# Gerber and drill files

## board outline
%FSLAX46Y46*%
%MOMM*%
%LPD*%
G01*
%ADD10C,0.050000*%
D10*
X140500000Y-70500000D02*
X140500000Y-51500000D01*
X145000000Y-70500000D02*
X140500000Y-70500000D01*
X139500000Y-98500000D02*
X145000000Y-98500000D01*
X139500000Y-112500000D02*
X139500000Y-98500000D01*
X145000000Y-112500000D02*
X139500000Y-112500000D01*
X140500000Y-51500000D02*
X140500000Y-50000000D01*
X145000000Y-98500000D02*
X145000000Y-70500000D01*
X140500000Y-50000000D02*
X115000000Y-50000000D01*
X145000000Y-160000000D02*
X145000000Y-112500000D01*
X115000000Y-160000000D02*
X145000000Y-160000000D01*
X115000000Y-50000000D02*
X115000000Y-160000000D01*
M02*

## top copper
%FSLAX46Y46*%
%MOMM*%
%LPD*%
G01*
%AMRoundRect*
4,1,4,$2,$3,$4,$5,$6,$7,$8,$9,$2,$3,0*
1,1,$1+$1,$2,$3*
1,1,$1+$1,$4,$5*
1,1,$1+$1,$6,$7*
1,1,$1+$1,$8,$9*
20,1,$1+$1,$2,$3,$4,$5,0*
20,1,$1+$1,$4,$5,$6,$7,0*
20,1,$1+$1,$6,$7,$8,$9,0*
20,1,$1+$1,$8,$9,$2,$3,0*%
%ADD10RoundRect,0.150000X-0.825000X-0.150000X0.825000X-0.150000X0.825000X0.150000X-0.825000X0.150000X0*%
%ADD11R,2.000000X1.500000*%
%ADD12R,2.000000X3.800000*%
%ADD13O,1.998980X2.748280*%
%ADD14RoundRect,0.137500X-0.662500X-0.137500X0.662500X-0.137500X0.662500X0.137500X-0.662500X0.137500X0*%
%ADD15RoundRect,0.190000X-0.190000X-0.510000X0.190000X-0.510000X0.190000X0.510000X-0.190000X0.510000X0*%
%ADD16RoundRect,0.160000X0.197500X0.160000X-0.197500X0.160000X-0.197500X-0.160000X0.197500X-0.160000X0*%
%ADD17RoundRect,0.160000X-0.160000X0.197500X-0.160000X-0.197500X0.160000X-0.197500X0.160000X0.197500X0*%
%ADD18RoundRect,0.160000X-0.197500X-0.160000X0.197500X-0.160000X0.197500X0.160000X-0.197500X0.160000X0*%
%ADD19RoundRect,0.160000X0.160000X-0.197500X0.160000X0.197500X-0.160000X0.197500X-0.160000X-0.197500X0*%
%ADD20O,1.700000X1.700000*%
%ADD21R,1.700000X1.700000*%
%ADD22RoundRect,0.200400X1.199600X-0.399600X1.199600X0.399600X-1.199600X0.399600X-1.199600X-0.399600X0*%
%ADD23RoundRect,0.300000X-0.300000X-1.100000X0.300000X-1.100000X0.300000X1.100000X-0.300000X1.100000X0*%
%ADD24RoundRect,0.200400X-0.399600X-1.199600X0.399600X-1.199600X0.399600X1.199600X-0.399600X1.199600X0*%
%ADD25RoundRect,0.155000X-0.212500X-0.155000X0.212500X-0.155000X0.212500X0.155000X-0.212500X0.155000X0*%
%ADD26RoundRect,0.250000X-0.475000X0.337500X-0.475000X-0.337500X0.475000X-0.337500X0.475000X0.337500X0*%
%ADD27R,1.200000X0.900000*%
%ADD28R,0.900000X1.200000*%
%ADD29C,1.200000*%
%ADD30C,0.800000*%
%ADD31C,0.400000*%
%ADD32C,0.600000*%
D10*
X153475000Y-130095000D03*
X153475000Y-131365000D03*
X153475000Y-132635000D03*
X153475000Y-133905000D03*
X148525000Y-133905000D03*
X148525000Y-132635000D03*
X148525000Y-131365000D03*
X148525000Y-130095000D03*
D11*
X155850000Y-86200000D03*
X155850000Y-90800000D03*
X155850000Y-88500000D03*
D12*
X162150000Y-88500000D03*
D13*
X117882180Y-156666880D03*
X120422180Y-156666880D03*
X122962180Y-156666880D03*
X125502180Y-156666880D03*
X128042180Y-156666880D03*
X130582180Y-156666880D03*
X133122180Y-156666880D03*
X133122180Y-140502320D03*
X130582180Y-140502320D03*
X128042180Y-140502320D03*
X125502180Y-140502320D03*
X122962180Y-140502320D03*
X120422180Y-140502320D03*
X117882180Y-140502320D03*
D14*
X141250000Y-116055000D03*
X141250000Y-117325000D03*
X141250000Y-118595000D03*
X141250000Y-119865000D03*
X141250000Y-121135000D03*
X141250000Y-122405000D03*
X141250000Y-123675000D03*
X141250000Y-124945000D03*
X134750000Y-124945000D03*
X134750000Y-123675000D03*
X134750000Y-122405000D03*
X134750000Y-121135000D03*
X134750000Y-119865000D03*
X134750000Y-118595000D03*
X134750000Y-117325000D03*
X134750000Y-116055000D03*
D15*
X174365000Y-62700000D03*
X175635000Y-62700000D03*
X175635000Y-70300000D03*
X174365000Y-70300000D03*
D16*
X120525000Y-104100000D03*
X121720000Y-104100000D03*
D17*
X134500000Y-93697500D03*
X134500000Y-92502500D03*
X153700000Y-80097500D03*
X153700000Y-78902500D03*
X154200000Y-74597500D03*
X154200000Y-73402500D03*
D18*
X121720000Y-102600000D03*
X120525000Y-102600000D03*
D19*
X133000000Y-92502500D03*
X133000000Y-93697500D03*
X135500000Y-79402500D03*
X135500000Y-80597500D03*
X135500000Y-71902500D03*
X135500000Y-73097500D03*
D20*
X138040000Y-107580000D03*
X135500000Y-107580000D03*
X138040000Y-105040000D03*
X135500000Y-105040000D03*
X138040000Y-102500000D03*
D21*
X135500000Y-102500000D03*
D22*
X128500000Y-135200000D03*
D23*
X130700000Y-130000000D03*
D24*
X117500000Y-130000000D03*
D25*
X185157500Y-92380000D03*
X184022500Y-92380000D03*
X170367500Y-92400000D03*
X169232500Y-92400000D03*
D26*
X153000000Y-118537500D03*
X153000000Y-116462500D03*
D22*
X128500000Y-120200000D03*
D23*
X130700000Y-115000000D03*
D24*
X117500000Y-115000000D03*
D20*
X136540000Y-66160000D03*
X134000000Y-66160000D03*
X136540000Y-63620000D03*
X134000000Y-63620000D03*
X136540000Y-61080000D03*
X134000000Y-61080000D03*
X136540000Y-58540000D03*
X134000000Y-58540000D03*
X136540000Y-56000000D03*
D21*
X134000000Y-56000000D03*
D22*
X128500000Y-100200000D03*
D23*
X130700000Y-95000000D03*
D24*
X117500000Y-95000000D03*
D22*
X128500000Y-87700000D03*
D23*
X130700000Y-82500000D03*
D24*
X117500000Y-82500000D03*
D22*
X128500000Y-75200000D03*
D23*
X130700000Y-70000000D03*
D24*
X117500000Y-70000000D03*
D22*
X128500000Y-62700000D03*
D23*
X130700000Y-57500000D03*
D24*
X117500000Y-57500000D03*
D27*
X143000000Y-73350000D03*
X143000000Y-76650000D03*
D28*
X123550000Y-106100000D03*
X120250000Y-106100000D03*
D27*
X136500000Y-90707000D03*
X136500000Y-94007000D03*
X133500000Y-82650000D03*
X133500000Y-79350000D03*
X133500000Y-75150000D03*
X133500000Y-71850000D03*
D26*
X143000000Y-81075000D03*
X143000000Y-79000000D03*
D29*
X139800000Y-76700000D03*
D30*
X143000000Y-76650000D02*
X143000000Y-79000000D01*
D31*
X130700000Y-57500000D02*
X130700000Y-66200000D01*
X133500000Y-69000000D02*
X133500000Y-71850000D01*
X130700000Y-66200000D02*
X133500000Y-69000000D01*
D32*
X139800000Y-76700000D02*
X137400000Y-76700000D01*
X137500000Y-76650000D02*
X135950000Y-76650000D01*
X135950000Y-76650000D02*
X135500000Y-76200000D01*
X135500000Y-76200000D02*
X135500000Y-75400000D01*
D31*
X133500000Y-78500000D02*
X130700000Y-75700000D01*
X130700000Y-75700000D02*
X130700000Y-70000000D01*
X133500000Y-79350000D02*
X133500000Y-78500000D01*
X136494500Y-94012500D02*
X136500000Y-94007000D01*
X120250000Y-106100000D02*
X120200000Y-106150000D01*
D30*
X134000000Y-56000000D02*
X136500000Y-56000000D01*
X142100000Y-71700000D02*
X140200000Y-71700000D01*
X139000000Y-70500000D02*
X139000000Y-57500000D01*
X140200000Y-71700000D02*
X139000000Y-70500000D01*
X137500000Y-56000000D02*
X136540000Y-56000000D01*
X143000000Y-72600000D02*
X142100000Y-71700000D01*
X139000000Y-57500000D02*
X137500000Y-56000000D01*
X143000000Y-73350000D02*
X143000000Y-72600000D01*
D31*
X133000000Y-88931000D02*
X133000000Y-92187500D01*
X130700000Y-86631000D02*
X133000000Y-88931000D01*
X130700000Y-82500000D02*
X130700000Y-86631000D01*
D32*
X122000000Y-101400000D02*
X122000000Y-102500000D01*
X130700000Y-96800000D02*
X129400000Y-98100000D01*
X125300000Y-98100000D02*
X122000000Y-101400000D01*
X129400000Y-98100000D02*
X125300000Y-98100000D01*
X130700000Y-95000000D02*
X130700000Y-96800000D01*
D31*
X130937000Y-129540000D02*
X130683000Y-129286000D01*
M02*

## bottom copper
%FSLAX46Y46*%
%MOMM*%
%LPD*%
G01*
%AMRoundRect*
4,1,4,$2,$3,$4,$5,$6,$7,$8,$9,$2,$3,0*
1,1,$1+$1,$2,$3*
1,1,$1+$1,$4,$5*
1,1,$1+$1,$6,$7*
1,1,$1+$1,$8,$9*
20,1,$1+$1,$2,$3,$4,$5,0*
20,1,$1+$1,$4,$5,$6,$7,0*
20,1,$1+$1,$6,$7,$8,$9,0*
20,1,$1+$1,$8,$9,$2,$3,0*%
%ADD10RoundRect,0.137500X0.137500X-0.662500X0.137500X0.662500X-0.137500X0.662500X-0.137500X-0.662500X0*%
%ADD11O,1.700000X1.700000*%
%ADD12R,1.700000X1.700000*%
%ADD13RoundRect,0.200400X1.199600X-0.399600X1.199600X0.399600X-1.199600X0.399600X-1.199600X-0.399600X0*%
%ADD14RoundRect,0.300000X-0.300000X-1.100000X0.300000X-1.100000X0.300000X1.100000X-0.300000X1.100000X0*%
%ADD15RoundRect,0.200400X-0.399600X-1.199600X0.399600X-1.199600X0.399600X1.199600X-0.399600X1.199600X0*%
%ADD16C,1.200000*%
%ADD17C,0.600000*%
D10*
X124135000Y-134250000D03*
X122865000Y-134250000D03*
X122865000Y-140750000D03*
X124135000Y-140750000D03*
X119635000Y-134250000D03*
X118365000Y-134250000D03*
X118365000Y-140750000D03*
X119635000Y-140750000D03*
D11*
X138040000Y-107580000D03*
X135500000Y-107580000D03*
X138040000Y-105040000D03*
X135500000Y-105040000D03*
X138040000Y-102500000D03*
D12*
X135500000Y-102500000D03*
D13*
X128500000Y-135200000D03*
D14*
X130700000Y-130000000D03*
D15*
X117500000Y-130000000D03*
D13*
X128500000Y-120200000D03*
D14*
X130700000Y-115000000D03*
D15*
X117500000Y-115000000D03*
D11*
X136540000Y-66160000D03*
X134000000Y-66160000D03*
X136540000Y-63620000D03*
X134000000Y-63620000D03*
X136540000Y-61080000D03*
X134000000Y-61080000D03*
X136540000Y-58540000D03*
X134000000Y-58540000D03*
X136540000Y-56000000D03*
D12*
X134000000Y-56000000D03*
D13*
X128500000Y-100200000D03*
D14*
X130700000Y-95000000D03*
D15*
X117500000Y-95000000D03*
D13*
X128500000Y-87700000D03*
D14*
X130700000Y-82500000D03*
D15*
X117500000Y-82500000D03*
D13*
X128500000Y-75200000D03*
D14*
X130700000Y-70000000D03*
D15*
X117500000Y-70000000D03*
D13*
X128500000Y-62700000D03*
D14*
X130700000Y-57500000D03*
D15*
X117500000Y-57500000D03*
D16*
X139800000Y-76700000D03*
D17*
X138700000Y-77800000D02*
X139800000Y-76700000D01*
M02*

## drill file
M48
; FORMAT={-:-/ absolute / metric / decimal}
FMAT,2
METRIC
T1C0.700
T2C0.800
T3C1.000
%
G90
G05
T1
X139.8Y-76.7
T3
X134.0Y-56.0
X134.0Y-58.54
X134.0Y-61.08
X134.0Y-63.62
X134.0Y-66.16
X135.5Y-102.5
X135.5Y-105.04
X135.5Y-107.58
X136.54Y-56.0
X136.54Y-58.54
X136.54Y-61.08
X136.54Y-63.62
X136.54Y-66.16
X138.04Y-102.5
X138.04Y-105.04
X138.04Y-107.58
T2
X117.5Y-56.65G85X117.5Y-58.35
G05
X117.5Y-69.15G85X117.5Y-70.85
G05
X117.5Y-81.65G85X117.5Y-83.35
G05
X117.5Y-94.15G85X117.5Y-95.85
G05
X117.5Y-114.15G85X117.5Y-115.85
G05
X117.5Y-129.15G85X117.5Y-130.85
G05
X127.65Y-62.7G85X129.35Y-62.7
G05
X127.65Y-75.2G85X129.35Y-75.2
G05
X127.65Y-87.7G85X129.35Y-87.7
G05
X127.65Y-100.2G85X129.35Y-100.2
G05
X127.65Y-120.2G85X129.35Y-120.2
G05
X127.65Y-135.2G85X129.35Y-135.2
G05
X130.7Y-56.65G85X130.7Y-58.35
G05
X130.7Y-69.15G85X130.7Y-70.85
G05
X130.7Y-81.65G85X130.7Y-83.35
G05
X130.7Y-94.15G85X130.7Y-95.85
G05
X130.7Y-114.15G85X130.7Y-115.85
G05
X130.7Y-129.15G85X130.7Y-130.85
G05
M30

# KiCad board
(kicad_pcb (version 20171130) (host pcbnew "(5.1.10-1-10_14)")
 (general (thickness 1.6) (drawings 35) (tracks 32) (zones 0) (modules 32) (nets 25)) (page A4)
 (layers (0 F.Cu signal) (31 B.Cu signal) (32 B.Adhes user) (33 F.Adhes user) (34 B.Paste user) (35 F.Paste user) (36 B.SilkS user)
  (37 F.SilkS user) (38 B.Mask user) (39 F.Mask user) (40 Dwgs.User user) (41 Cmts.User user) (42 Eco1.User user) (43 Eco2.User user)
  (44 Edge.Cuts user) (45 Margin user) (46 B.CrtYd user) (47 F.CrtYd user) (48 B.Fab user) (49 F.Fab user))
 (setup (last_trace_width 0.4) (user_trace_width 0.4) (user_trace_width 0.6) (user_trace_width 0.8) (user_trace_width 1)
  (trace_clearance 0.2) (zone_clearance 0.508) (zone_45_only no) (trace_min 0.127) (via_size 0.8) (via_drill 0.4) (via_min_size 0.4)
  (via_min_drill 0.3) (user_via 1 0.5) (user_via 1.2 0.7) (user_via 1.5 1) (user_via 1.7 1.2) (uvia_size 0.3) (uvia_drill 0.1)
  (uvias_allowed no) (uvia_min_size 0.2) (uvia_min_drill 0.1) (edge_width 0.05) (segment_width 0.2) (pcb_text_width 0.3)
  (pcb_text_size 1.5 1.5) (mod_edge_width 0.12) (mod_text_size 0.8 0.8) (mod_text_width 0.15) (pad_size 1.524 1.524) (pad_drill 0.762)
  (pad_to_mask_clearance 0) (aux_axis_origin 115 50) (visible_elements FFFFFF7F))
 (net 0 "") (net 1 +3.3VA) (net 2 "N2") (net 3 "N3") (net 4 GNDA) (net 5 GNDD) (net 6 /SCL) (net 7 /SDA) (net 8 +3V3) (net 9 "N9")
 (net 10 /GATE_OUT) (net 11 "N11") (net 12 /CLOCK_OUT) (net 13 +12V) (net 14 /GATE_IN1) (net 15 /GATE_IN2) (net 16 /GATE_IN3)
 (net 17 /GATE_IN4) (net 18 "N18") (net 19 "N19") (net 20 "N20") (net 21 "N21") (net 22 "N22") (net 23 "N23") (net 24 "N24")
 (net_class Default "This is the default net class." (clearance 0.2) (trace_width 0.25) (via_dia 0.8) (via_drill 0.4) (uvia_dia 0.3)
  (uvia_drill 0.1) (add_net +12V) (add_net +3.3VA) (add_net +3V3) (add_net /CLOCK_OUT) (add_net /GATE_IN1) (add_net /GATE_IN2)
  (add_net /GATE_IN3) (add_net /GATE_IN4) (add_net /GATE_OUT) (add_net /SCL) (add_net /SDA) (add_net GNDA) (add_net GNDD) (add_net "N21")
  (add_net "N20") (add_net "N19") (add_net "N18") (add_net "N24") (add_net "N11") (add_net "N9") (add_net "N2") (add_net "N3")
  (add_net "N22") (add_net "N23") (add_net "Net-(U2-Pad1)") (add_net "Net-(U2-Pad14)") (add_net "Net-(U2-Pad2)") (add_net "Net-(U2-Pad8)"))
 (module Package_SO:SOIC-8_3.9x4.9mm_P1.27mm (layer F.Cu) (at 151 132)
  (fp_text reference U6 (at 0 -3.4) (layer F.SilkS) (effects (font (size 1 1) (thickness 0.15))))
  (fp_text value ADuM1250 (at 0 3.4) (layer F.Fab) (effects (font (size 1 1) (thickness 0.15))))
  (pad 8 smd roundrect (at 2.475 -1.905) (size 1.95 0.6) (layers F.Cu F.Paste F.Mask) (roundrect_rratio 0.25) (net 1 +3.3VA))
  (pad 7 smd roundrect (at 2.475 -0.635) (size 1.95 0.6) (layers F.Cu F.Paste F.Mask) (roundrect_rratio 0.25) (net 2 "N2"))
  (pad 6 smd roundrect (at 2.475 0.635) (size 1.95 0.6) (layers F.Cu F.Paste F.Mask) (roundrect_rratio 0.25) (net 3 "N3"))
  (pad 5 smd roundrect (at 2.475 1.905) (size 1.95 0.6) (layers F.Cu F.Paste F.Mask) (roundrect_rratio 0.25) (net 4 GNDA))
  (pad 4 smd roundrect (at -2.475 1.905) (size 1.95 0.6) (layers F.Cu F.Paste F.Mask) (roundrect_rratio 0.25) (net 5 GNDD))
  (pad 3 smd roundrect (at -2.475 0.635) (size 1.95 0.6) (layers F.Cu F.Paste F.Mask) (roundrect_rratio 0.25) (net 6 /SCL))
  (pad 2 smd roundrect (at -2.475 -0.635) (size 1.95 0.6) (layers F.Cu F.Paste F.Mask) (roundrect_rratio 0.25) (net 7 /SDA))
  (pad 1 smd roundrect (at -2.475 -1.905) (size 1.95 0.6) (layers F.Cu F.Paste F.Mask) (roundrect_rratio 0.25) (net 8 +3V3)))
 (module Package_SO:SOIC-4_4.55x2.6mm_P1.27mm (layer B.Cu) (at 123.5 137.5 90)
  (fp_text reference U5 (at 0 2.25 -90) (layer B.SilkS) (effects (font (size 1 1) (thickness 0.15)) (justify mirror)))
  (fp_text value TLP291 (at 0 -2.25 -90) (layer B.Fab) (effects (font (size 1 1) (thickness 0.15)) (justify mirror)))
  (pad 4 smd roundrect (at 3.25 0.635 90) (size 1.6 0.55) (layers B.Cu B.Paste B.Mask) (roundrect_rratio 0.25) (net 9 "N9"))
  (pad 3 smd roundrect (at 3.25 -0.635 90) (size 1.6 0.55) (layers B.Cu B.Paste B.Mask) (roundrect_rratio 0.25) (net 4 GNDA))
  (pad 2 smd roundrect (at -3.25 -0.635 90) (size 1.6 0.55) (layers B.Cu B.Paste B.Mask) (roundrect_rratio 0.25) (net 5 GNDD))
  (pad 1 smd roundrect (at -3.25 0.635 90) (size 1.6 0.55) (layers B.Cu B.Paste B.Mask) (roundrect_rratio 0.25) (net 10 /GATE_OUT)))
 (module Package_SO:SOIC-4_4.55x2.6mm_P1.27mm (layer B.Cu) (at 119 137.5 90)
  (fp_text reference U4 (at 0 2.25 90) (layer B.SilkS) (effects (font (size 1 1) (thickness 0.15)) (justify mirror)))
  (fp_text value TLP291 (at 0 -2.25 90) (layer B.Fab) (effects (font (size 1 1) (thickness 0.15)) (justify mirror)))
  (pad 4 smd roundrect (at 3.25 0.635 90) (size 1.6 0.55) (layers B.Cu B.Paste B.Mask) (roundrect_rratio 0.25) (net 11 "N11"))
  (pad 3 smd roundrect (at 3.25 -0.635 90) (size 1.6 0.55) (layers B.Cu B.Paste B.Mask) (roundrect_rratio 0.25) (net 4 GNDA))
  (pad 2 smd roundrect (at -3.25 -0.635 90) (size 1.6 0.55) (layers B.Cu B.Paste B.Mask) (roundrect_rratio 0.25) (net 5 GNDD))
  (pad 1 smd roundrect (at -3.25 0.635 90) (size 1.6 0.55) (layers B.Cu B.Paste B.Mask) (roundrect_rratio 0.25) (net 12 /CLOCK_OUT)))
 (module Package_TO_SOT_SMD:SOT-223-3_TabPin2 (layer F.Cu) (at 159 88.5)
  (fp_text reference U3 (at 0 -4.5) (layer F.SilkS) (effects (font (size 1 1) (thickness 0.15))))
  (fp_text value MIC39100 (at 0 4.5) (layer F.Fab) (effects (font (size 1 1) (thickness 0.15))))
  (pad 1 smd rect (at -3.15 -2.3) (size 2 1.5) (layers F.Cu F.Paste F.Mask) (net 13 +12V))
  (pad 3 smd rect (at -3.15 2.3) (size 2 1.5) (layers F.Cu F.Paste F.Mask) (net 1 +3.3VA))
  (pad 2 smd rect (at -3.15 0) (size 2 1.5) (layers F.Cu F.Paste F.Mask) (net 4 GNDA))
  (pad 2 smd rect (at 3.15 0) (size 2 3.8) (layers F.Cu F.Paste F.Mask) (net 4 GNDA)))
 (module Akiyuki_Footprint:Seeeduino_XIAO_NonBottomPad (layer F.Cu) (at 136 157.5 90)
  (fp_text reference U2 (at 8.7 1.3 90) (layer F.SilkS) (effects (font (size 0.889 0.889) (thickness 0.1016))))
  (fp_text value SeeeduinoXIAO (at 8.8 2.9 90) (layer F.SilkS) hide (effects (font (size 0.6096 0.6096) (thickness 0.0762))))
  (pad "" smd circle (at 10.238803 -16.264187 180) (size 1.143 1.143) (layers Dwgs.User))
  (pad "" smd circle (at 7.698803 -16.264187 180) (size 1.143 1.143) (layers Dwgs.User))
  (pad "" smd circle (at 10.238803 -18.804187 180) (size 1.143 1.143) (layers Dwgs.User))
  (pad "" smd circle (at 7.698803 -18.804187 180) (size 1.143 1.143) (layers Dwgs.User))
  (pad "" smd oval (at 10.25 -1.8 180) (size 2.032 1.016) (layers Dwgs.User))
  (pad "" smd oval (at 7.7 -1.8 180) (size 2.032 1.016) (layers Dwgs.User))
  (pad 1 smd oval (at 0.83312 -18.11782 90) (size 2.74828 1.99898) (layers F.Cu F.Paste F.Mask))
  (pad 2 smd oval (at 0.83312 -15.57782 90) (size 2.74828 1.99898) (layers F.Cu F.Paste F.Mask))
  (pad 3 smd oval (at 0.83312 -13.03782 90) (size 2.74828 1.99898) (layers F.Cu F.Paste F.Mask) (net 12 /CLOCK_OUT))
  (pad 4 smd oval (at 0.83312 -10.49782 90) (size 2.74828 1.99898) (layers F.Cu F.Paste F.Mask) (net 10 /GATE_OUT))
  (pad 5 smd oval (at 0.83312 -7.95782 90) (size 2.74828 1.99898) (layers F.Cu F.Paste F.Mask) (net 7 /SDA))
  (pad 6 smd oval (at 0.83312 -5.41782 90) (size 2.74828 1.99898) (layers F.Cu F.Paste F.Mask) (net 6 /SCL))
  (pad 7 smd oval (at 0.83312 -2.87782 90) (size 2.74828 1.99898) (layers F.Cu F.Paste F.Mask) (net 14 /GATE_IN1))
  (pad 8 smd oval (at 16.99768 -2.87782 90) (size 2.74828 1.99898) (layers F.Cu F.Paste F.Mask))
  (pad 9 smd oval (at 16.99768 -5.41782 90) (size 2.74828 1.99898) (layers F.Cu F.Paste F.Mask) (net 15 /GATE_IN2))
  (pad 10 smd oval (at 16.99768 -7.95782 90) (size 2.74828 1.99898) (layers F.Cu F.Paste F.Mask) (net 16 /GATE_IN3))
  (pad 11 smd oval (at 16.99768 -10.49782 90) (size 2.74828 1.99898) (layers F.Cu F.Paste F.Mask) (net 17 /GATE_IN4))
  (pad 12 smd oval (at 16.99768 -13.03782 90) (size 2.74828 1.99898) (layers F.Cu F.Paste F.Mask) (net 8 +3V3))
  (pad 13 smd oval (at 16.99768 -15.57782 90) (size 2.74828 1.99898) (layers F.Cu F.Paste F.Mask) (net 5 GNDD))
  (pad 14 smd oval (at 16.99768 -18.11782 90) (size 2.74828 1.99898) (layers F.Cu F.Paste F.Mask)))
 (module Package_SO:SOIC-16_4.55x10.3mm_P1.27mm (layer F.Cu) (at 138 120.5)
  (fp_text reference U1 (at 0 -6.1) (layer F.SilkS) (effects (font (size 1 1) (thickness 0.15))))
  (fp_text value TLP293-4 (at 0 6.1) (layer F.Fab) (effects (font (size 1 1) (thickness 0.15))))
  (pad 16 smd roundrect (at 3.25 -4.445) (size 1.6 0.55) (layers F.Cu F.Paste F.Mask) (roundrect_rratio 0.25) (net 14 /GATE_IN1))
  (pad 15 smd roundrect (at 3.25 -3.175) (size 1.6 0.55) (layers F.Cu F.Paste F.Mask) (roundrect_rratio 0.25) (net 5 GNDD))
  (pad 14 smd roundrect (at 3.25 -1.905) (size 1.6 0.55) (layers F.Cu F.Paste F.Mask) (roundrect_rratio 0.25) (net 15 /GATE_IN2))
  (pad 13 smd roundrect (at 3.25 -0.635) (size 1.6 0.55) (layers F.Cu F.Paste F.Mask) (roundrect_rratio 0.25) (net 5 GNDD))
  (pad 12 smd roundrect (at 3.25 0.635) (size 1.6 0.55) (layers F.Cu F.Paste F.Mask) (roundrect_rratio 0.25) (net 16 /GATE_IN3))
  (pad 11 smd roundrect (at 3.25 1.905) (size 1.6 0.55) (layers F.Cu F.Paste F.Mask) (roundrect_rratio 0.25) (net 5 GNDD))
  (pad 10 smd roundrect (at 3.25 3.175) (size 1.6 0.55) (layers F.Cu F.Paste F.Mask) (roundrect_rratio 0.25) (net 17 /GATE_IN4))
  (pad 9 smd roundrect (at 3.25 4.445) (size 1.6 0.55) (layers F.Cu F.Paste F.Mask) (roundrect_rratio 0.25) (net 5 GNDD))
  (pad 8 smd roundrect (at -3.25 4.445) (size 1.6 0.55) (layers F.Cu F.Paste F.Mask) (roundrect_rratio 0.25) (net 4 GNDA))
  (pad 7 smd roundrect (at -3.25 3.175) (size 1.6 0.55) (layers F.Cu F.Paste F.Mask) (roundrect_rratio 0.25) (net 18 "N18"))
  (pad 6 smd roundrect (at -3.25 1.905) (size 1.6 0.55) (layers F.Cu F.Paste F.Mask) (roundrect_rratio 0.25) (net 4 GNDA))
  (pad 5 smd roundrect (at -3.25 0.635) (size 1.6 0.55) (layers F.Cu F.Paste F.Mask) (roundrect_rratio 0.25) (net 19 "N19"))
  (pad 4 smd roundrect (at -3.25 -0.635) (size 1.6 0.55) (layers F.Cu F.Paste F.Mask) (roundrect_rratio 0.25) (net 4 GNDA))
  (pad 3 smd roundrect (at -3.25 -1.905) (size 1.6 0.55) (layers F.Cu F.Paste F.Mask) (roundrect_rratio 0.25) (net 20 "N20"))
  (pad 2 smd roundrect (at -3.25 -3.175) (size 1.6 0.55) (layers F.Cu F.Paste F.Mask) (roundrect_rratio 0.25) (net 4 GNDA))
  (pad 1 smd roundrect (at -3.25 -4.445) (size 1.6 0.55) (layers F.Cu F.Paste F.Mask) (roundrect_rratio 0.25) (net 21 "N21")))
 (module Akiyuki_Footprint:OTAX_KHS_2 (layer F.Cu) (at 175 66.5) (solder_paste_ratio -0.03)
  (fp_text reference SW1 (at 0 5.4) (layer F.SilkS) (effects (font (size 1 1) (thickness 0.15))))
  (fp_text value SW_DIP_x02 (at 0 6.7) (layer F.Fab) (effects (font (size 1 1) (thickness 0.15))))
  (pad 4 smd roundrect (at -0.635 -3.8) (size 0.76 1.4) (layers F.Cu F.Paste F.Mask) (roundrect_rratio 0.25) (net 3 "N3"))
  (pad 3 smd roundrect (at 0.635 -3.8) (size 0.76 1.4) (layers F.Cu F.Paste F.Mask) (roundrect_rratio 0.25) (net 2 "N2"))
  (pad 2 smd roundrect (at 0.635 3.8) (size 0.76 1.4) (layers F.Cu F.Paste F.Mask) (roundrect_rratio 0.25) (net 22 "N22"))
  (pad 1 smd roundrect (at -0.635 3.8) (size 0.76 1.4) (layers F.Cu F.Paste F.Mask) (roundrect_rratio 0.25) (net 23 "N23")))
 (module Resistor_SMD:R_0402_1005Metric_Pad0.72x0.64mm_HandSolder (layer F.Cu) (at 121.1225 104.1 180)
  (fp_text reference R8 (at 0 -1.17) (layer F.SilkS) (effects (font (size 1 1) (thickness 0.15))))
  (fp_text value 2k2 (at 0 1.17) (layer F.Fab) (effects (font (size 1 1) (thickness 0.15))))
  (pad 2 smd roundrect (at 0.5975 0 180) (size 0.715 0.64) (layers F.Cu F.Paste F.Mask) (roundrect_rratio 0.25) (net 23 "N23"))
  (pad 1 smd roundrect (at -0.5975 0 180) (size 0.715 0.64) (layers F.Cu F.Paste F.Mask) (roundrect_rratio 0.25) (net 1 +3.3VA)))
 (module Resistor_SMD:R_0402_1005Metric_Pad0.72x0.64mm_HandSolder (layer F.Cu) (at 134.5 93.1 270)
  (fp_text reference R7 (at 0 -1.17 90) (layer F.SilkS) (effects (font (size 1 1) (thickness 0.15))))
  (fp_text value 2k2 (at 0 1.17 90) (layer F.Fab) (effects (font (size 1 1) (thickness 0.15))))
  (pad 2 smd roundrect (at 0.5975 0 270) (size 0.715 0.64) (layers F.Cu F.Paste F.Mask) (roundrect_rratio 0.25) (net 22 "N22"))
  (pad 1 smd roundrect (at -0.5975 0 270) (size 0.715 0.64) (layers F.Cu F.Paste F.Mask) (roundrect_rratio 0.25) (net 1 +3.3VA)))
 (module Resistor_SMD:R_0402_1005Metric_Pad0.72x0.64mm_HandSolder (layer F.Cu) (at 153.7 79.5 270)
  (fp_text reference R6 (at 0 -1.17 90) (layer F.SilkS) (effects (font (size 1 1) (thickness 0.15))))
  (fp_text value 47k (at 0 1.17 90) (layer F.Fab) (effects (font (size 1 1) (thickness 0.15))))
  (pad 2 smd roundrect (at 0.5975 0 270) (size 0.715 0.64) (layers F.Cu F.Paste F.Mask) (roundrect_rratio 0.25) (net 13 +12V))
  (pad 1 smd roundrect (at -0.5975 0 270) (size 0.715 0.64) (layers F.Cu F.Paste F.Mask) (roundrect_rratio 0.25) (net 9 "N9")))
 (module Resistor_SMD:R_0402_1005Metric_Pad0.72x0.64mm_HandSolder (layer F.Cu) (at 154.2 74 270)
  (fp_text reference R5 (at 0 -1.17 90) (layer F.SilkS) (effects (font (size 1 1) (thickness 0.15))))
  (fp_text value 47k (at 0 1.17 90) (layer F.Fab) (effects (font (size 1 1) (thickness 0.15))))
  (pad 2 smd roundrect (at 0.5975 0 270) (size 0.715 0.64) (layers F.Cu F.Paste F.Mask) (roundrect_rratio 0.25) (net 13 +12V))
  (pad 1 smd roundrect (at -0.5975 0 270) (size 0.715 0.64) (layers F.Cu F.Paste F.Mask) (roundrect_rratio 0.25) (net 11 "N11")))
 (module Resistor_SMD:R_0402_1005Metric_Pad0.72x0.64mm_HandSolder (layer F.Cu) (at 121.1225 102.6)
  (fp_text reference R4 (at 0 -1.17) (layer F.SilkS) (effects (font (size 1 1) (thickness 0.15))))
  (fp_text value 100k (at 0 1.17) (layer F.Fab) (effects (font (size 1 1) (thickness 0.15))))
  (pad 2 smd roundrect (at 0.5975 0) (size 0.715 0.64) (layers F.Cu F.Paste F.Mask) (roundrect_rratio 0.25) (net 18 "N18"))
  (pad 1 smd roundrect (at -0.5975 0) (size 0.715 0.64) (layers F.Cu F.Paste F.Mask) (roundrect_rratio 0.25) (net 4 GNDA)))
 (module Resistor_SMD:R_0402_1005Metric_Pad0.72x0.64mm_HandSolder (layer F.Cu) (at 133 93.1 90)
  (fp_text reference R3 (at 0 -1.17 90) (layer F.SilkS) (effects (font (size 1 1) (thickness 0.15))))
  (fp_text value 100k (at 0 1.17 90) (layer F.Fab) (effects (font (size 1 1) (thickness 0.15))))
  (pad 2 smd roundrect (at 0.5975 0 90) (size 0.715 0.64) (layers F.Cu F.Paste F.Mask) (roundrect_rratio 0.25) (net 19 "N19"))
  (pad 1 smd roundrect (at -0.5975 0 90) (size 0.715 0.64) (layers F.Cu F.Paste F.Mask) (roundrect_rratio 0.25) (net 4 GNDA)))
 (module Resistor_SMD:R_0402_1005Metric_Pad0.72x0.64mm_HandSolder (layer F.Cu) (at 135.5 80 90)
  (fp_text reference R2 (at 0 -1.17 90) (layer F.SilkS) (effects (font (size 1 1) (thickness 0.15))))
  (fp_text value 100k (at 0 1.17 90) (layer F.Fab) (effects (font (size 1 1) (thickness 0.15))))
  (pad 2 smd roundrect (at 0.5975 0 90) (size 0.715 0.64) (layers F.Cu F.Paste F.Mask) (roundrect_rratio 0.25) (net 20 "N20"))
  (pad 1 smd roundrect (at -0.5975 0 90) (size 0.715 0.64) (layers F.Cu F.Paste F.Mask) (roundrect_rratio 0.25) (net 4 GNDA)))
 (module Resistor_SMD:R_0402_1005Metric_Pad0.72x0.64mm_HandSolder (layer F.Cu) (at 135.5 72.5 90)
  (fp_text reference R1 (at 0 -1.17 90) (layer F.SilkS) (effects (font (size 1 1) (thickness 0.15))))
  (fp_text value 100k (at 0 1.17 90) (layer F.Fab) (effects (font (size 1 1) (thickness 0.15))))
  (pad 2 smd roundrect (at 0.5975 0 90) (size 0.715 0.64) (layers F.Cu F.Paste F.Mask) (roundrect_rratio 0.25) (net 21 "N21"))
  (pad 1 smd roundrect (at -0.5975 0 90) (size 0.715 0.64) (layers F.Cu F.Paste F.Mask) (roundrect_rratio 0.25) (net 4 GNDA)))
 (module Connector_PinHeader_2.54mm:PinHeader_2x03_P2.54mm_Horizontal (layer F.Cu) (at 135.5 102.5)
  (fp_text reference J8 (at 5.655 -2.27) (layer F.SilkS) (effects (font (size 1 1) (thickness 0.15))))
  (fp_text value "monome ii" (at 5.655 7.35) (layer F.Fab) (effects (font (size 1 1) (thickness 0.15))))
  (pad 6 thru_hole oval (at 2.54 5.08) (size 1.7 1.7) (drill 1) (layers *.Cu *.Mask) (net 4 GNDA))
  (pad 5 thru_hole oval (at 0 5.08) (size 1.7 1.7) (drill 1) (layers *.Cu *.Mask) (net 4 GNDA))
  (pad 4 thru_hole oval (at 2.54 2.54) (size 1.7 1.7) (drill 1) (layers *.Cu *.Mask) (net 3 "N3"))
  (pad 3 thru_hole oval (at 0 2.54) (size 1.7 1.7) (drill 1) (layers *.Cu *.Mask) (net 3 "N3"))
  (pad 2 thru_hole oval (at 2.54 0) (size 1.7 1.7) (drill 1) (layers *.Cu *.Mask) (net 2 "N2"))
  (pad 1 thru_hole rect (at 0 0) (size 1.7 1.7) (drill 1) (layers *.Cu *.Mask) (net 2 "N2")))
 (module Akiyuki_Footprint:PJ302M (layer F.Cu) (at 115 130)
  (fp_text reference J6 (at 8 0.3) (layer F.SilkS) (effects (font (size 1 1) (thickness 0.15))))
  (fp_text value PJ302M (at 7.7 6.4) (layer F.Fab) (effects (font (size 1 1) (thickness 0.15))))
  (pad 2 thru_hole roundrect (at 13.5 5.2 90) (size 1.2 2.8) (drill oval 0.8 2.5) (layers *.Cu *.Mask) (roundrect_rratio 0.167) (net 4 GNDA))
  (pad 3 thru_hole roundrect (at 15.7 0) (size 1.2 2.8) (drill oval 0.8 2.5) (layers *.Cu *.Mask) (roundrect_rratio 0.25) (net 11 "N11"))
  (pad 1 thru_hole roundrect (at 2.5 0) (size 1.2 2.8) (drill oval 0.8 2.5) (layers *.Cu *.Mask) (roundrect_rratio 0.167) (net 4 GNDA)))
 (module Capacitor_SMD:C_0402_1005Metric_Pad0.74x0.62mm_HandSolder (layer F.Cu) (at 184.59 92.38)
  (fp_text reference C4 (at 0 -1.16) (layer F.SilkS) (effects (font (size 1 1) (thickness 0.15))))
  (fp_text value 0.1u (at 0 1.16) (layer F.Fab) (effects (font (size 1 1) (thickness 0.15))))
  (pad 2 smd roundrect (at 0.5675 0) (size 0.735 0.62) (layers F.Cu F.Paste F.Mask) (roundrect_rratio 0.25) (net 1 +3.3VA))
  (pad 1 smd roundrect (at -0.5675 0) (size 0.735 0.62) (layers F.Cu F.Paste F.Mask) (roundrect_rratio 0.25) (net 4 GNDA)))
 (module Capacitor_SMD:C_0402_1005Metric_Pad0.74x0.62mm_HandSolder (layer F.Cu) (at 169.8 92.4)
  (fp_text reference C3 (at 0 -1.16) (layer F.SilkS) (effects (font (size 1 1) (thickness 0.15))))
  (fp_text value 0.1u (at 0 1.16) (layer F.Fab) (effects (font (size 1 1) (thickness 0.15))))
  (pad 2 smd roundrect (at 0.5675 0) (size 0.735 0.62) (layers F.Cu F.Paste F.Mask) (roundrect_rratio 0.25) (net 5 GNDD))
  (pad 1 smd roundrect (at -0.5675 0) (size 0.735 0.62) (layers F.Cu F.Paste F.Mask) (roundrect_rratio 0.25) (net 8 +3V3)))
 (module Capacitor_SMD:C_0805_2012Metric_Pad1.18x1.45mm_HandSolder (layer F.Cu) (at 153 117.5 270)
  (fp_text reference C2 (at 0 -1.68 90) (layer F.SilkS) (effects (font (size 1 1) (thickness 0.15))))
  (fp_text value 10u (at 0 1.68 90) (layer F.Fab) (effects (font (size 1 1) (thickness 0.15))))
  (pad 2 smd roundrect (at 1.0375 0 270) (size 1.175 1.45) (layers F.Cu F.Paste F.Mask) (roundrect_rratio 0.212766) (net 4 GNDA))
  (pad 1 smd roundrect (at -1.0375 0 270) (size 1.175 1.45) (layers F.Cu F.Paste F.Mask) (roundrect_rratio 0.212766) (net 1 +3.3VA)))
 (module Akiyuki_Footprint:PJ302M (layer F.Cu) (at 115 115)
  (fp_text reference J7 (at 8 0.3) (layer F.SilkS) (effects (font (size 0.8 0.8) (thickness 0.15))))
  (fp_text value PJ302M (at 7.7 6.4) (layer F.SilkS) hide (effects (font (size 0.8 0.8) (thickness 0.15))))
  (pad 2 thru_hole roundrect (at 13.5 5.2 90) (size 1.2 2.8) (drill oval 0.8 2.5) (layers *.Cu *.Mask) (roundrect_rratio 0.167) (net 4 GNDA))
  (pad 3 thru_hole roundrect (at 15.7 0) (size 1.2 2.8) (drill oval 0.8 2.5) (layers *.Cu *.Mask) (roundrect_rratio 0.25) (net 9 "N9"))
  (pad 1 thru_hole roundrect (at 2.5 0) (size 1.2 2.8) (drill oval 0.8 2.5) (layers *.Cu *.Mask) (roundrect_rratio 0.167) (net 4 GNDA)))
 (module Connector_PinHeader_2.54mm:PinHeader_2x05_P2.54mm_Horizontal (layer F.Cu) (at 134 56)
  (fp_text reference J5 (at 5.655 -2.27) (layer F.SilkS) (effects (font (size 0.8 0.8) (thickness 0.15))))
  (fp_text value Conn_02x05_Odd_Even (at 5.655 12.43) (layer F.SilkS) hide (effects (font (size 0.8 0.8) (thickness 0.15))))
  (pad 10 thru_hole oval (at 2.54 10.16) (size 1.7 1.7) (drill 1) (layers *.Cu *.Mask))
  (pad 9 thru_hole oval (at 0 10.16) (size 1.7 1.7) (drill 1) (layers *.Cu *.Mask))
  (pad 8 thru_hole oval (at 2.54 7.62) (size 1.7 1.7) (drill 1) (layers *.Cu *.Mask) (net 4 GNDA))
  (pad 7 thru_hole oval (at 0 7.62) (size 1.7 1.7) (drill 1) (layers *.Cu *.Mask) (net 4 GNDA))
  (pad 6 thru_hole oval (at 2.54 5.08) (size 1.7 1.7) (drill 1) (layers *.Cu *.Mask) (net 4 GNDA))
  (pad 5 thru_hole oval (at 0 5.08) (size 1.7 1.7) (drill 1) (layers *.Cu *.Mask) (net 4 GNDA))
  (pad 4 thru_hole oval (at 2.54 2.54) (size 1.7 1.7) (drill 1) (layers *.Cu *.Mask) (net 4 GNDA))
  (pad 3 thru_hole oval (at 0 2.54) (size 1.7 1.7) (drill 1) (layers *.Cu *.Mask) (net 4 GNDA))
  (pad 2 thru_hole oval (at 2.54 0) (size 1.7 1.7) (drill 1) (layers *.Cu *.Mask) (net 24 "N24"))
  (pad 1 thru_hole rect (at 0 0) (size 1.7 1.7) (drill 1) (layers *.Cu *.Mask) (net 24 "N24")))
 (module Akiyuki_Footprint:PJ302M (layer F.Cu) (at 115 95)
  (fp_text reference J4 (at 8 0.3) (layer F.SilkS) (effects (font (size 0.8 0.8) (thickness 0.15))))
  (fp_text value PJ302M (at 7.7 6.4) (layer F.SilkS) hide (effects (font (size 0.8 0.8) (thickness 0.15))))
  (pad 2 thru_hole roundrect (at 13.5 5.2 90) (size 1.2 2.8) (drill oval 0.8 2.5) (layers *.Cu *.Mask) (roundrect_rratio 0.167) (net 4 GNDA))
  (pad 3 thru_hole roundrect (at 15.7 0) (size 1.2 2.8) (drill oval 0.8 2.5) (layers *.Cu *.Mask) (roundrect_rratio 0.25) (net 18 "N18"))
  (pad 1 thru_hole roundrect (at 2.5 0) (size 1.2 2.8) (drill oval 0.8 2.5) (layers *.Cu *.Mask) (roundrect_rratio 0.167) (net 4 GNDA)))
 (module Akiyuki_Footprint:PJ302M (layer F.Cu) (at 115 82.5)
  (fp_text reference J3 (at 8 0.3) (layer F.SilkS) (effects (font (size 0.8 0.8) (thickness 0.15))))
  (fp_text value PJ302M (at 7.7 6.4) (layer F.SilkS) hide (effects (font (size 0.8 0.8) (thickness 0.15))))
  (pad 2 thru_hole roundrect (at 13.5 5.2 90) (size 1.2 2.8) (drill oval 0.8 2.5) (layers *.Cu *.Mask) (roundrect_rratio 0.167) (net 4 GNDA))
  (pad 3 thru_hole roundrect (at 15.7 0) (size 1.2 2.8) (drill oval 0.8 2.5) (layers *.Cu *.Mask) (roundrect_rratio 0.25) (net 19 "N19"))
  (pad 1 thru_hole roundrect (at 2.5 0) (size 1.2 2.8) (drill oval 0.8 2.5) (layers *.Cu *.Mask) (roundrect_rratio 0.167) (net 4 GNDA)))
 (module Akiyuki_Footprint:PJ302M (layer F.Cu) (at 115 70)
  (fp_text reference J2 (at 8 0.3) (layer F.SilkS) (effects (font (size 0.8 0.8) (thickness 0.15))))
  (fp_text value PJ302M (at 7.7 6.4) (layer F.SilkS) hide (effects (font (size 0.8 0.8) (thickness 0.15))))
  (pad 2 thru_hole roundrect (at 13.5 5.2 90) (size 1.2 2.8) (drill oval 0.8 2.5) (layers *.Cu *.Mask) (roundrect_rratio 0.167) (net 4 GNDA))
  (pad 3 thru_hole roundrect (at 15.7 0) (size 1.2 2.8) (drill oval 0.8 2.5) (layers *.Cu *.Mask) (roundrect_rratio 0.25) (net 20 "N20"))
  (pad 1 thru_hole roundrect (at 2.5 0) (size 1.2 2.8) (drill oval 0.8 2.5) (layers *.Cu *.Mask) (roundrect_rratio 0.167) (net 4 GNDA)))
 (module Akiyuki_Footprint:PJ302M (layer F.Cu) (at 115 57.5)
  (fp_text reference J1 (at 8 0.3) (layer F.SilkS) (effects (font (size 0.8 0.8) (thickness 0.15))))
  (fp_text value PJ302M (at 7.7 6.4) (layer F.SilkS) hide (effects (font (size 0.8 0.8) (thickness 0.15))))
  (pad 2 thru_hole roundrect (at 13.5 5.2 90) (size 1.2 2.8) (drill oval 0.8 2.5) (layers *.Cu *.Mask) (roundrect_rratio 0.167) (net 4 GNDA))
  (pad 3 thru_hole roundrect (at 15.7 0) (size 1.2 2.8) (drill oval 0.8 2.5) (layers *.Cu *.Mask) (roundrect_rratio 0.25) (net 21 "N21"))
  (pad 1 thru_hole roundrect (at 2.5 0) (size 1.2 2.8) (drill oval 0.8 2.5) (layers *.Cu *.Mask) (roundrect_rratio 0.167) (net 4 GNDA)))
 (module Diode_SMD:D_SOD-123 (layer F.Cu) (at 143 75 90)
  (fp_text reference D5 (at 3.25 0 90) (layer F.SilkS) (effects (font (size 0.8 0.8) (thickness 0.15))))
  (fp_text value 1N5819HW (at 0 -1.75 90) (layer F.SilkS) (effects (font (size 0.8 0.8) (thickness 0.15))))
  (pad 2 smd rect (at 1.65 0 90) (size 0.9 1.2) (layers F.Cu F.Paste F.Mask) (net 24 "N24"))
  (pad 1 smd rect (at -1.65 0 90) (size 0.9 1.2) (layers F.Cu F.Paste F.Mask) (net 13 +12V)))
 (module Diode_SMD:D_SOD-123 (layer F.Cu) (at 121.9 106.1)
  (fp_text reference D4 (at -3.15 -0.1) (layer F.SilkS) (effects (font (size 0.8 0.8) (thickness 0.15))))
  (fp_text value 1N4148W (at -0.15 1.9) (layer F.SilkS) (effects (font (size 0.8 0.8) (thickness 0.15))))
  (pad 2 smd rect (at 1.65 0) (size 0.9 1.2) (layers F.Cu F.Paste F.Mask) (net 4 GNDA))
  (pad 1 smd rect (at -1.65 0) (size 0.9 1.2) (layers F.Cu F.Paste F.Mask) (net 18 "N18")))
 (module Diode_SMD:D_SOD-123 (layer F.Cu) (at 136.5 92.357 90)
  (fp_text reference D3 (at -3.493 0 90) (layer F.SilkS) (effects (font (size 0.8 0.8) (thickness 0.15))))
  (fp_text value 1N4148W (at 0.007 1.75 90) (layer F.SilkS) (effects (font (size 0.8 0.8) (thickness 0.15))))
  (pad 2 smd rect (at 1.65 0 90) (size 0.9 1.2) (layers F.Cu F.Paste F.Mask) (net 4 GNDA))
  (pad 1 smd rect (at -1.65 0 90) (size 0.9 1.2) (layers F.Cu F.Paste F.Mask) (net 19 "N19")))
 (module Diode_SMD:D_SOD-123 (layer F.Cu) (at 133.5 81 270)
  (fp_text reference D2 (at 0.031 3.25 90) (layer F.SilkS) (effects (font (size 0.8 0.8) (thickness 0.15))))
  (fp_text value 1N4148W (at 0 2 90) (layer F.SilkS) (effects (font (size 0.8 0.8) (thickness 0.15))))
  (pad 2 smd rect (at 1.65 0 270) (size 0.9 1.2) (layers F.Cu F.Paste F.Mask) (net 4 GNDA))
  (pad 1 smd rect (at -1.65 0 270) (size 0.9 1.2) (layers F.Cu F.Paste F.Mask) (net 20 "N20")))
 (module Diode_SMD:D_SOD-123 (layer F.Cu) (at 133.5 73.5 270)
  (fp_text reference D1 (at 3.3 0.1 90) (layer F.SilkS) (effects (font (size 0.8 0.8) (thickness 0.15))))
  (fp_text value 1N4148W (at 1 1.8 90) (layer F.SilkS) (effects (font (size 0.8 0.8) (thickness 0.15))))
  (pad 2 smd rect (at 1.65 0 270) (size 0.9 1.2) (layers F.Cu F.Paste F.Mask) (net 4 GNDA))
  (pad 1 smd rect (at -1.65 0 270) (size 0.9 1.2) (layers F.Cu F.Paste F.Mask) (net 21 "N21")))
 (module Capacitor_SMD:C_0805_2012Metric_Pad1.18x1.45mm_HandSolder (layer F.Cu) (at 143 80.0375 270)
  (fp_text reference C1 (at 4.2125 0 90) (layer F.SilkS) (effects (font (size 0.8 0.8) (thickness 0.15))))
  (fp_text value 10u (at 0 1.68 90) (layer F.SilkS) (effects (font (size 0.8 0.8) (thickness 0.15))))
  (pad 2 smd roundrect (at 1.0375 0 270) (size 1.175 1.45) (layers F.Cu F.Paste F.Mask) (roundrect_rratio 0.2127659574468085) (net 4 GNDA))
  (pad 1 smd roundrect (at -1.0375 0 270) (size 1.175 1.45) (layers F.Cu F.Paste F.Mask) (roundrect_rratio 0.2127659574468085) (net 13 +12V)))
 (gr_line (start 140.5 70.5) (end 140.5 51.5) (layer Edge.Cuts) (width 0.05))
 (gr_line (start 145 70.5) (end 140.5 70.5) (layer Edge.Cuts) (width 0.05))
 (gr_line (start 139.5 98.5) (end 145 98.5) (layer Edge.Cuts) (width 0.05))
 (gr_line (start 139.5 112.5) (end 139.5 98.5) (layer Edge.Cuts) (width 0.05))
 (gr_line (start 145 112.5) (end 139.5 112.5) (layer Edge.Cuts) (width 0.05))
 (gr_line (start 140.5 51.5) (end 140.5 50) (layer Edge.Cuts) (width 0.05))
 (gr_line (start 145 98.5) (end 145 70.5) (layer Edge.Cuts) (width 0.05))
 (gr_line (start 140.5 50) (end 115 50) (layer Edge.Cuts) (width 0.05))
 (gr_line (start 145 160) (end 145 112.5) (layer Edge.Cuts) (width 0.05))
 (gr_line (start 115 160) (end 145 160) (layer Edge.Cuts) (width 0.05))
 (gr_line (start 115 50) (end 115 160) (layer Edge.Cuts) (width 0.05))
 (segment (start 143 76.65) (end 143 79) (width 0.8) (layer F.Cu) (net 13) (status 30))
 (segment (start 130.7 57.5) (end 130.7 66.2) (width 0.4) (layer F.Cu) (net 21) (status 10))
 (segment (start 133.5 69) (end 133.5 71.85) (width 0.4) (layer F.Cu) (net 21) (status 20))
 (segment (start 130.7 66.2) (end 133.5 69) (width 0.4) (layer F.Cu) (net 21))
 (via (at 139.8 76.7) (size 1.2) (drill 0.7) (layers F.Cu B.Cu) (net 4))
 (segment (start 139.8 76.7) (end 137.4 76.7) (width 0.6) (layer F.Cu) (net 4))
 (segment (start 137.5 76.65) (end 135.95 76.65) (width 0.6) (layer F.Cu) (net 4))
 (segment (start 135.95 76.65) (end 135.5 76.2) (width 0.6) (layer F.Cu) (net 4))
 (segment (start 135.5 76.2) (end 135.5 75.4) (width 0.6) (layer F.Cu) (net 4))
 (segment (start 138.7 77.8) (end 139.8 76.7) (width 0.6) (layer B.Cu) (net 4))
 (segment (start 133.5 78.5) (end 130.7 75.7) (width 0.4) (layer F.Cu) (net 20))
 (segment (start 130.7 75.7) (end 130.7 70) (width 0.4) (layer F.Cu) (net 20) (status 20))
 (segment (start 133.5 79.35) (end 133.5 78.5) (width 0.4) (layer F.Cu) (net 20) (status 10))
 (segment (start 136.4945 94.0125) (end 136.5 94.007) (width 0.4) (layer F.Cu) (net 19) (status 30))
 (segment (start 120.25 106.1) (end 120.2 106.15) (width 0.4) (layer F.Cu) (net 18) (status 30))
 (segment (start 134 56) (end 136.5 56) (width 0.8) (layer F.Cu) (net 24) (status 30))
 (segment (start 142.1 71.7) (end 140.2 71.7) (width 0.8) (layer F.Cu) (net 24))
 (segment (start 139 70.5) (end 139 57.5) (width 0.8) (layer F.Cu) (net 24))
 (segment (start 140.2 71.7) (end 139 70.5) (width 0.8) (layer F.Cu) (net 24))
 (segment (start 137.5 56) (end 136.54 56) (width 0.8) (layer F.Cu) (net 24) (status 20))
 (segment (start 143 72.6) (end 142.1 71.7) (width 0.8) (layer F.Cu) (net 24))
 (segment (start 139 57.5) (end 137.5 56) (width 0.8) (layer F.Cu) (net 24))
 (segment (start 143 73.35) (end 143 72.6) (width 0.8) (layer F.Cu) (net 24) (status 10))
 (segment (start 133 88.931) (end 133 92.1875) (width 0.4) (layer F.Cu) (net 19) (status 20))
 (segment (start 130.7 86.631) (end 133 88.931) (width 0.4) (layer F.Cu) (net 19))
 (segment (start 130.7 82.5) (end 130.7 86.631) (width 0.4) (layer F.Cu) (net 19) (status 10))
 (segment (start 122 101.4) (end 122 102.5) (width 0.6) (layer F.Cu) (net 18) (status 20))
 (segment (start 130.7 96.8) (end 129.4 98.1) (width 0.6) (layer F.Cu) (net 18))
 (segment (start 125.3 98.1) (end 122 101.4) (width 0.6) (layer F.Cu) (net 18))
 (segment (start 129.4 98.1) (end 125.3 98.1) (width 0.6) (layer F.Cu) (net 18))
 (segment (start 130.7 95) (end 130.7 96.8) (width 0.6) (layer F.Cu) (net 18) (status 10))
 (segment (start 130.937 129.54) (end 130.683 129.286) (width 0.4) (layer F.Cu) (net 11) (status 30)))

